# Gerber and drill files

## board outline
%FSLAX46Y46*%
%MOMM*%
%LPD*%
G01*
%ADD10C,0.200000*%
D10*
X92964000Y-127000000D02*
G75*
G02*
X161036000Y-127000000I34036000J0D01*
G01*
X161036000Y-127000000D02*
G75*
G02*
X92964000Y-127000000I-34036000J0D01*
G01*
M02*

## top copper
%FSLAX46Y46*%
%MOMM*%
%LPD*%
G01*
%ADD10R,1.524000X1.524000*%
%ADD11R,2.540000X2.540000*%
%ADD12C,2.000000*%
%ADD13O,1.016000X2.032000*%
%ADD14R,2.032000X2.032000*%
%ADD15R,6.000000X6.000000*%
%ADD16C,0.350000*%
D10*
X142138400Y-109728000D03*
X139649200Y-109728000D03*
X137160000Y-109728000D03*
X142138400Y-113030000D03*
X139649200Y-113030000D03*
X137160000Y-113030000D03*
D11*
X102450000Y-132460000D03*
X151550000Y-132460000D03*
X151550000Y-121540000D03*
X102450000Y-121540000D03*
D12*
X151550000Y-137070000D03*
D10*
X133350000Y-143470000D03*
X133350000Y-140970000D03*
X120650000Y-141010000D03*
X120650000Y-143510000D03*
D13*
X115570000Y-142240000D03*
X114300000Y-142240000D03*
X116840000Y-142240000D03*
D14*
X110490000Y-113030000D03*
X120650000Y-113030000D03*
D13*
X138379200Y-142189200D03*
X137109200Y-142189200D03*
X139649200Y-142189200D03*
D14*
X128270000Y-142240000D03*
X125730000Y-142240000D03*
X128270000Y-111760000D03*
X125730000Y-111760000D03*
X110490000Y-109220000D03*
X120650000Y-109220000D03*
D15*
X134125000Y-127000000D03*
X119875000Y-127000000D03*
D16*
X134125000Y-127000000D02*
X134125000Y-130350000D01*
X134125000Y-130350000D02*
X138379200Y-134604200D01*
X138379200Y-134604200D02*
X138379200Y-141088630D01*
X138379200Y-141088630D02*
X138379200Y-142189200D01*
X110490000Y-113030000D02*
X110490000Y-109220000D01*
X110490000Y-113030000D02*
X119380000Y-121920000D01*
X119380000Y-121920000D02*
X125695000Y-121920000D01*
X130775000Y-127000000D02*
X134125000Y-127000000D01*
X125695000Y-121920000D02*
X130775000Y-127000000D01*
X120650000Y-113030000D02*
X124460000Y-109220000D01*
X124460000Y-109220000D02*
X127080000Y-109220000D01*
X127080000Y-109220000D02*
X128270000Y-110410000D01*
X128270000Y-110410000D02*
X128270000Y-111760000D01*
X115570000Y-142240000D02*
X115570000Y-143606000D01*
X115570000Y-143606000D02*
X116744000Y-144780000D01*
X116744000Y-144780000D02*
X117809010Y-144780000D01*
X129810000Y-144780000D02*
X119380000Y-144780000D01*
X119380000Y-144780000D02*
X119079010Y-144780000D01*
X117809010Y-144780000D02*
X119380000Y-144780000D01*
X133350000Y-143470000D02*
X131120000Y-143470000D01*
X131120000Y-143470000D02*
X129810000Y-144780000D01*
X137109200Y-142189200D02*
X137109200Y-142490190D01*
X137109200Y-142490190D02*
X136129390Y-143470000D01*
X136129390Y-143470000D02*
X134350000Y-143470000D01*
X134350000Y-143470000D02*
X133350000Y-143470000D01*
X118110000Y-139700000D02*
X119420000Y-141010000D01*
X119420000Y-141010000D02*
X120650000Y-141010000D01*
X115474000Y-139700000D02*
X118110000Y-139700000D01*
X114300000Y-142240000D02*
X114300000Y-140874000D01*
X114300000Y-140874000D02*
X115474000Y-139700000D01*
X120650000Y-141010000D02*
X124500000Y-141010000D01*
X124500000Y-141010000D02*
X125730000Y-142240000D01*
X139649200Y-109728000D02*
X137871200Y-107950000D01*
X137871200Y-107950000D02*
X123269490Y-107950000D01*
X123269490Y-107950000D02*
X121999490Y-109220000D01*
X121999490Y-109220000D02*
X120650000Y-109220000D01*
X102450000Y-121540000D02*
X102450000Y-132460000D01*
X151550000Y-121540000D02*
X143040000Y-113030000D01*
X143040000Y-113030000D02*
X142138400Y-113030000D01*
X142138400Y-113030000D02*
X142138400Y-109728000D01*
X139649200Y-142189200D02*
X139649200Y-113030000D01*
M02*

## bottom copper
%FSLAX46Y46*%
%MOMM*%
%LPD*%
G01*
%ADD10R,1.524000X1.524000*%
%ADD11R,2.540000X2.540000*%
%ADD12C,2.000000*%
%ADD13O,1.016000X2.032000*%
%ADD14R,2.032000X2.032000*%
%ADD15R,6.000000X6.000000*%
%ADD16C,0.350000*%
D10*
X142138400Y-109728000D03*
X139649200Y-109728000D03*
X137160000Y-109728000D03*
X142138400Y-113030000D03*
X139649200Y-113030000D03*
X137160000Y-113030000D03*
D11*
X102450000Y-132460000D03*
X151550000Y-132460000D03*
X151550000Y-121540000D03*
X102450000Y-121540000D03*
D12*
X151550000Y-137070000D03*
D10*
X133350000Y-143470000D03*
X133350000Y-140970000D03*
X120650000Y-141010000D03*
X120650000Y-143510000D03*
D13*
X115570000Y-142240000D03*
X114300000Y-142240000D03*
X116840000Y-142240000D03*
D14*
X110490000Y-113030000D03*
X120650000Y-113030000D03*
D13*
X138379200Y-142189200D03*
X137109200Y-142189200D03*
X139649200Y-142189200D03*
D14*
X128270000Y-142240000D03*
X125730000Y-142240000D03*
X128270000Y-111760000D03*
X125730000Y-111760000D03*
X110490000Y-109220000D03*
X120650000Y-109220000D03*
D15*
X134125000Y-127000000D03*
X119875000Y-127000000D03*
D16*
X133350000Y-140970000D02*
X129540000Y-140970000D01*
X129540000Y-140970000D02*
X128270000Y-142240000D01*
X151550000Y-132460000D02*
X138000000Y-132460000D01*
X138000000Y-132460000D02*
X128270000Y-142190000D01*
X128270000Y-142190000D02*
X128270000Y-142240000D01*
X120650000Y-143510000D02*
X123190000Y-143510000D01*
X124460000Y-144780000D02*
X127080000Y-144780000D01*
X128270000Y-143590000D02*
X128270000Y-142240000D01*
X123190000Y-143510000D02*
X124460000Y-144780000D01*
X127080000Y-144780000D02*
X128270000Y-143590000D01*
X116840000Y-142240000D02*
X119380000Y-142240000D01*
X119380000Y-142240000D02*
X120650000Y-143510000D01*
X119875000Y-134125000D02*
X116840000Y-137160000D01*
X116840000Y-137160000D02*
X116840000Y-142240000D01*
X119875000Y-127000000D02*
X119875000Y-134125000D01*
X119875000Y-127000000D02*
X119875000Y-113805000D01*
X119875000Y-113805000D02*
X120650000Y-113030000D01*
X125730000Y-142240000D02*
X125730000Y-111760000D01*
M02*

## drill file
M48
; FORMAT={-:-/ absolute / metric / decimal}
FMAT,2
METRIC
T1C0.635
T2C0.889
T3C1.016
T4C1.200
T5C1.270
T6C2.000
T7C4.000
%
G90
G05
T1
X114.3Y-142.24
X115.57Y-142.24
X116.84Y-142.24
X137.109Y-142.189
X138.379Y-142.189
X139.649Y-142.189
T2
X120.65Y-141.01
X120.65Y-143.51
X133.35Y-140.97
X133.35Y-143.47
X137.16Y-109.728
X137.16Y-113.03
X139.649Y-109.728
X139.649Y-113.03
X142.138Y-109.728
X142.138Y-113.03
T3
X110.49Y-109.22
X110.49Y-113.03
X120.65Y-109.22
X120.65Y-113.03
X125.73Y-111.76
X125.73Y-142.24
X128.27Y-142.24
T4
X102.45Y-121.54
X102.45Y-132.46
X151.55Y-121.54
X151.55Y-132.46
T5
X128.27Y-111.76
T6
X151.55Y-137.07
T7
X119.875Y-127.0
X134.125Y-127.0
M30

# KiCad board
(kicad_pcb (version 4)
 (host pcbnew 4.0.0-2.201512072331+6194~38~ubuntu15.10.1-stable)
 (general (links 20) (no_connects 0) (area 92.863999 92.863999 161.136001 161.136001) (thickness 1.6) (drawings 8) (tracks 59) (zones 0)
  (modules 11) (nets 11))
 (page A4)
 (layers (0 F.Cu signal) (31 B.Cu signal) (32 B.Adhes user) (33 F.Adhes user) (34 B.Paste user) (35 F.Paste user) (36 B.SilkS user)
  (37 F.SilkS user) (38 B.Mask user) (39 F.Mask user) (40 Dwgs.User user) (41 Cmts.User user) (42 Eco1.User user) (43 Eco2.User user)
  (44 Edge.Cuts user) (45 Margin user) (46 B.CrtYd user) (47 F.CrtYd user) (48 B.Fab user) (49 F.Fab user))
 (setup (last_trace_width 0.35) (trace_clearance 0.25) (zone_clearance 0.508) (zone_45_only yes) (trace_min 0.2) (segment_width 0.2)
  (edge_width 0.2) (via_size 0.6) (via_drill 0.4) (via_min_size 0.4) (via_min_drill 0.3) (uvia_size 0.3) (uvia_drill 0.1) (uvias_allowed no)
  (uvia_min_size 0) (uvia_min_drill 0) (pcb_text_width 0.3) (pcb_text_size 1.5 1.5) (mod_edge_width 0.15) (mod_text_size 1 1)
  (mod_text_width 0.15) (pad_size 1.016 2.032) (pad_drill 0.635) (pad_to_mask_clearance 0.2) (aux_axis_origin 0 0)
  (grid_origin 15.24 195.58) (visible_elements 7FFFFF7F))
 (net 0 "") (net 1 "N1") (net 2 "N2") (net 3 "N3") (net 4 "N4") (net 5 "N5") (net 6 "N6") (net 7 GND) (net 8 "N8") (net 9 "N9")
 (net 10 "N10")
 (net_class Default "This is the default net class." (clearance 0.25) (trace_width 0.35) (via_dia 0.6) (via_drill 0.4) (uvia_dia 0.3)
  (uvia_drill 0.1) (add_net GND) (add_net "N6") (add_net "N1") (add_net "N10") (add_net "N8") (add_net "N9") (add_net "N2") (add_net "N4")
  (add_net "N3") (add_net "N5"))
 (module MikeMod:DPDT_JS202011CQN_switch (layer F.Cu) (at 139.6492 111.379 180)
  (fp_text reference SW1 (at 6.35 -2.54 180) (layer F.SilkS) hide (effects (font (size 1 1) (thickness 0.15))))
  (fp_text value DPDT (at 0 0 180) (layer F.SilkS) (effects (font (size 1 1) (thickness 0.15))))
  (pad 1 thru_hole rect (at -2.4892 1.651 180) (size 1.524 1.524) (drill 0.889) (layers *.Cu F.SilkS F.Mask) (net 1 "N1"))
  (pad 2 thru_hole rect (at 0 1.651 180) (size 1.524 1.524) (drill 0.889) (layers *.Cu F.SilkS F.Mask) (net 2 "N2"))
  (pad 3 thru_hole rect (at 2.4892 1.651 180) (size 1.524 1.524) (drill 0.889) (layers *.Cu F.SilkS F.Mask) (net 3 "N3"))
  (pad 4 thru_hole rect (at -2.4892 -1.651 180) (size 1.524 1.524) (drill 0.889) (layers *.Cu F.SilkS F.Mask) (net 1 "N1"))
  (pad 5 thru_hole rect (at 0 -1.651 180) (size 1.524 1.524) (drill 0.889) (layers *.Cu F.SilkS F.Mask) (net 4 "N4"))
  (pad 6 thru_hole rect (at 2.4892 -1.651 180) (size 1.524 1.524) (drill 0.889) (layers *.Cu F.SilkS F.Mask) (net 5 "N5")))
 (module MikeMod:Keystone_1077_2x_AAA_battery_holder (layer F.Cu) (at 127 127 180)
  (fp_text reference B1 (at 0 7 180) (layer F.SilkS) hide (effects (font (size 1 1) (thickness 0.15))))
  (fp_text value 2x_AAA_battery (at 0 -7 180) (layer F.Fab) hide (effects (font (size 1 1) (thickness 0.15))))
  (pad 1 thru_hole rect (at 24.55 -5.46 180) (size 2.54 2.54) (drill 1.2) (layers *.Cu F.SilkS F.Mask) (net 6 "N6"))
  (pad 2 thru_hole rect (at -24.55 -5.46 180) (size 2.54 2.54) (drill 1.2) (layers *.Cu F.SilkS F.Mask) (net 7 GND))
  (pad 3 thru_hole rect (at -24.55 5.46 180) (size 2.54 2.54) (drill 1.2) (layers *.Cu F.SilkS F.Mask) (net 1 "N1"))
  (pad 4 thru_hole rect (at 24.55 5.46 180) (size 2.54 2.54) (drill 1.2) (layers *.Cu F.SilkS F.Mask) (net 6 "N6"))
  (pad "" thru_hole circle (at -24.55 -10.07 180) (size 2 2) (drill 2) (layers *.Cu)))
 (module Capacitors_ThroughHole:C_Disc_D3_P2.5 (layer F.Cu) (at 133.35 143.47 90)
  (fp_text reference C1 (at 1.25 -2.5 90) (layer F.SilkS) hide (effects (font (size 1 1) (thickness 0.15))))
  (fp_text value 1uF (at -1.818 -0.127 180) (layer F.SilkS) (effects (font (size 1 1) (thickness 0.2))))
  (pad 1 thru_hole rect (at 0 0 90) (size 1.524 1.524) (drill 0.889) (layers *.Cu F.SilkS F.Mask) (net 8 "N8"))
  (pad 2 thru_hole rect (at 2.5 0 90) (size 1.524 1.524) (drill 0.889) (layers *.Cu F.SilkS F.Mask) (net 7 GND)))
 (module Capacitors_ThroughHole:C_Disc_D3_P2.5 (layer F.Cu) (at 120.65 141.01 270)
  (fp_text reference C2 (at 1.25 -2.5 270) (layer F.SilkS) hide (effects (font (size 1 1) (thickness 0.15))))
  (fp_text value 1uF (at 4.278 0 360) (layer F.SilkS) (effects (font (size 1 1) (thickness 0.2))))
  (pad 1 thru_hole rect (at 0 0 270) (size 1.524 1.524) (drill 0.889) (layers *.Cu F.SilkS F.Mask) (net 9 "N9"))
  (pad 2 thru_hole rect (at 2.5 0 270) (size 1.524 1.524) (drill 0.889) (layers *.Cu F.SilkS F.Mask) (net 7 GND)))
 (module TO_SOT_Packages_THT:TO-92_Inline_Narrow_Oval (layer F.Cu) (at 116.84 142.24 180)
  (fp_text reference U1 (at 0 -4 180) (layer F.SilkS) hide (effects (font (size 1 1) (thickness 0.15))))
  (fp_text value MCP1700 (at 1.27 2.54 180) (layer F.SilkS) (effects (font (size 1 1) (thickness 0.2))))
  (pad 2 thru_hole oval (at 1.27 0) (size 1.016 2.032) (drill 0.635) (layers *.Cu F.SilkS F.Mask) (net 8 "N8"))
  (pad 3 thru_hole oval (at 2.54 0) (size 1.016 2.032) (drill 0.635) (layers *.Cu F.SilkS F.Mask) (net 9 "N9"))
  (pad 1 thru_hole oval (at 0 0) (size 1.016 2.032) (drill 0.635) (layers *.Cu F.SilkS F.Mask) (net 7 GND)))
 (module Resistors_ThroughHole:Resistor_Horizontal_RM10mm (layer F.Cu) (at 115.57 113.03)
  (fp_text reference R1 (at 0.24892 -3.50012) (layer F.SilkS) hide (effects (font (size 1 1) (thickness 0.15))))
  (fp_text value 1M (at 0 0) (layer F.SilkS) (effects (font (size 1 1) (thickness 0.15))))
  (pad 1 thru_hole rect (at -5.08 0) (size 2.032 2.032) (drill 1.016) (layers *.Cu F.SilkS F.Mask) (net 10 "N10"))
  (pad 2 thru_hole rect (at 5.08 0) (size 2.032 2.032) (drill 1.016) (layers *.Cu F.SilkS F.Mask) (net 7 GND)))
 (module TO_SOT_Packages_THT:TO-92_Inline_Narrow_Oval (layer F.Cu) (at 139.6492 142.1892 180)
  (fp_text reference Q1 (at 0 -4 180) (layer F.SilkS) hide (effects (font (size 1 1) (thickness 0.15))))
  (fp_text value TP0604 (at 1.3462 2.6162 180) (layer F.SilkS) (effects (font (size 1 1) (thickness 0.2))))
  (pad 2 thru_hole oval (at 1.27 0) (size 1.016 2.032) (drill 0.635) (layers *.Cu F.SilkS F.Mask) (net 10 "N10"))
  (pad 3 thru_hole oval (at 2.54 0) (size 1.016 2.032) (drill 0.635) (layers *.Cu F.SilkS F.Mask) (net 8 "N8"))
  (pad 1 thru_hole oval (at 0 0) (size 1.016 2.032) (drill 0.635) (layers *.Cu F.SilkS F.Mask) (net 4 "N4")))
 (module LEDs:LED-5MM (layer F.Cu) (at 128.27 142.24 180)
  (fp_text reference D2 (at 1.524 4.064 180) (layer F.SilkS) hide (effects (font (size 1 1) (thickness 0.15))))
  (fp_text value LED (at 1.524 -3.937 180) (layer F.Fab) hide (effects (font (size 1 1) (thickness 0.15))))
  (pad 1 thru_hole rect (at 0 0 270) (size 2.032 2.032) (drill 1.016) (layers *.Cu F.SilkS F.Mask) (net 7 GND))
  (pad 2 thru_hole rect (at 2.54 0 180) (size 2.032 2.032) (drill 1.016) (layers *.Cu F.SilkS F.Mask) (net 9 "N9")))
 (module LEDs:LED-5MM (layer F.Cu) (at 128.27 111.76 180)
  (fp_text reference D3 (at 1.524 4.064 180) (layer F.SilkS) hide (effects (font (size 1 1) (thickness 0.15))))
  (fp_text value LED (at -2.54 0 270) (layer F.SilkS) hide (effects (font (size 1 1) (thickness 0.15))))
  (pad 1 thru_hole rect (at 0 0 270) (size 2.032 2.032) (drill 1.27) (layers *.Cu F.SilkS F.Mask) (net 7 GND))
  (pad 2 thru_hole rect (at 2.54 0 180) (size 2.032 2.032) (drill 1.016) (layers *.Cu F.SilkS F.Mask) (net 9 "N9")))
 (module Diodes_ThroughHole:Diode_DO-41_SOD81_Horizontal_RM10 (layer F.Cu) (at 120.65 109.21746 180)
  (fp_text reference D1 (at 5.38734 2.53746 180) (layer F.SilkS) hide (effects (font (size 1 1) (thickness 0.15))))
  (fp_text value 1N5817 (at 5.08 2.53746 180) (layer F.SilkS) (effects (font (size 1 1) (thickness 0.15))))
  (pad 2 thru_hole rect (at 10.16 -0.00254) (size 2.032 2.032) (drill 1.016) (layers *.Cu F.SilkS F.Mask) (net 10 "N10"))
  (pad 1 thru_hole rect (at 0 -0.00254) (size 2.032 2.032) (drill 1.016) (layers *.Cu F.SilkS F.Mask) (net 2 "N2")))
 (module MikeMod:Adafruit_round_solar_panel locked (layer B.Cu) (at 127 127)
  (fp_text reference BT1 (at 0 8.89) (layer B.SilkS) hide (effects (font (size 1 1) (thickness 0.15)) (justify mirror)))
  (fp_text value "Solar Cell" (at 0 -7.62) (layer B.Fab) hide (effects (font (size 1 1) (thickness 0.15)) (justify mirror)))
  (pad 1 thru_hole rect (at 7.125 0) (size 6 6) (drill 4) (layers *.Cu B.SilkS B.Mask) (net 10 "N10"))
  (pad 2 thru_hole rect (at -7.125 0) (size 6 6) (drill 4) (layers *.Cu B.SilkS B.Mask) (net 7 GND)))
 (gr_arc (start 127 127) (end 92.964 127) (angle 180) (layer Edge.Cuts) (width 0.2))
 (gr_arc (start 127 127) (end 161.036 127) (angle 180) (layer Edge.Cuts) (width 0.2))
 (segment (start 134.125 127) (end 134.125 130.35) (width 0.35) (layer F.Cu) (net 10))
 (segment (start 134.125 130.35) (end 138.3792 134.6042) (width 0.35) (layer F.Cu) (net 10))
 (segment (start 138.3792 134.6042) (end 138.3792 141.08863) (width 0.35) (layer F.Cu) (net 10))
 (segment (start 138.3792 141.08863) (end 138.3792 142.1892) (width 0.35) (layer F.Cu) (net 10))
 (segment (start 110.49 113.03) (end 110.49 109.22) (width 0.35) (layer F.Cu) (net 10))
 (segment (start 110.49 113.03) (end 119.38 121.92) (width 0.35) (layer F.Cu) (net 10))
 (segment (start 119.38 121.92) (end 125.695 121.92) (width 0.35) (layer F.Cu) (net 10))
 (segment (start 130.775 127) (end 134.125 127) (width 0.35) (layer F.Cu) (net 10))
 (segment (start 125.695 121.92) (end 130.775 127) (width 0.35) (layer F.Cu) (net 10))
 (segment (start 133.35 140.97) (end 129.54 140.97) (width 0.35) (layer B.Cu) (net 7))
 (segment (start 129.54 140.97) (end 128.27 142.24) (width 0.35) (layer B.Cu) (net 7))
 (segment (start 120.65 113.03) (end 124.46 109.22) (width 0.35) (layer F.Cu) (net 7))
 (segment (start 124.46 109.22) (end 127.08 109.22) (width 0.35) (layer F.Cu) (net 7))
 (segment (start 127.08 109.22) (end 128.27 110.41) (width 0.35) (layer F.Cu) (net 7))
 (segment (start 128.27 110.41) (end 128.27 111.76) (width 0.35) (layer F.Cu) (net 7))
 (segment (start 151.55 132.46) (end 138 132.46) (width 0.35) (layer B.Cu) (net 7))
 (segment (start 138 132.46) (end 128.27 142.19) (width 0.35) (layer B.Cu) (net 7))
 (segment (start 128.27 142.19) (end 128.27 142.24) (width 0.35) (layer B.Cu) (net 7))
 (segment (start 120.65 143.51) (end 123.19 143.51) (width 0.35) (layer B.Cu) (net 7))
 (segment (start 124.46 144.78) (end 127.08 144.78) (width 0.35) (layer B.Cu) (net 7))
 (segment (start 128.27 143.59) (end 128.27 142.24) (width 0.35) (layer B.Cu) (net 7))
 (segment (start 123.19 143.51) (end 124.46 144.78) (width 0.35) (layer B.Cu) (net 7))
 (segment (start 127.08 144.78) (end 128.27 143.59) (width 0.35) (layer B.Cu) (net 7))
 (segment (start 116.84 142.24) (end 119.38 142.24) (width 0.35) (layer B.Cu) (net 7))
 (segment (start 119.38 142.24) (end 120.65 143.51) (width 0.35) (layer B.Cu) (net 7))
 (segment (start 119.875 134.125) (end 116.84 137.16) (width 0.35) (layer B.Cu) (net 7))
 (segment (start 116.84 137.16) (end 116.84 142.24) (width 0.35) (layer B.Cu) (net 7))
 (segment (start 119.875 127) (end 119.875 134.125) (width 0.35) (layer B.Cu) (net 7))
 (segment (start 119.875 127) (end 119.875 113.805) (width 0.35) (layer B.Cu) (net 7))
 (segment (start 119.875 113.805) (end 120.65 113.03) (width 0.35) (layer B.Cu) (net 7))
 (segment (start 115.57 142.24) (end 115.57 143.606) (width 0.35) (layer F.Cu) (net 8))
 (segment (start 115.57 143.606) (end 116.744 144.78) (width 0.35) (layer F.Cu) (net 8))
 (segment (start 116.744 144.78) (end 117.80901 144.78) (width 0.35) (layer F.Cu) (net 8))
 (segment (start 129.81 144.78) (end 119.38 144.78) (width 0.35) (layer F.Cu) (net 8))
 (segment (start 119.38 144.78) (end 119.07901 144.78) (width 0.35) (layer F.Cu) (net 8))
 (segment (start 117.80901 144.78) (end 119.38 144.78) (width 0.35) (layer F.Cu) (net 8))
 (segment (start 133.35 143.47) (end 131.12 143.47) (width 0.35) (layer F.Cu) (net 8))
 (segment (start 131.12 143.47) (end 129.81 144.78) (width 0.35) (layer F.Cu) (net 8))
 (segment (start 137.1092 142.1892) (end 137.1092 142.49019) (width 0.35) (layer F.Cu) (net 8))
 (segment (start 137.1092 142.49019) (end 136.12939 143.47) (width 0.35) (layer F.Cu) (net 8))
 (segment (start 136.12939 143.47) (end 134.35 143.47) (width 0.35) (layer F.Cu) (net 8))
 (segment (start 134.35 143.47) (end 133.35 143.47) (width 0.35) (layer F.Cu) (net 8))
 (segment (start 118.11 139.7) (end 119.42 141.01) (width 0.35) (layer F.Cu) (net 9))
 (segment (start 119.42 141.01) (end 120.65 141.01) (width 0.35) (layer F.Cu) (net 9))
 (segment (start 115.474 139.7) (end 118.11 139.7) (width 0.35) (layer F.Cu) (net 9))
 (segment (start 114.3 142.24) (end 114.3 140.874) (width 0.35) (layer F.Cu) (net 9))
 (segment (start 114.3 140.874) (end 115.474 139.7) (width 0.35) (layer F.Cu) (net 9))
 (segment (start 120.65 141.01) (end 124.5 141.01) (width 0.35) (layer F.Cu) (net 9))
 (segment (start 125.73 142.24) (end 125.73 111.76) (width 0.35) (layer B.Cu) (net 9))
 (segment (start 124.5 141.01) (end 125.73 142.24) (width 0.35) (layer F.Cu) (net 9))
 (segment (start 139.6492 109.728) (end 137.8712 107.95) (width 0.35) (layer F.Cu) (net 2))
 (segment (start 137.8712 107.95) (end 123.26949 107.95) (width 0.35) (layer F.Cu) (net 2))
 (segment (start 123.26949 107.95) (end 121.99949 109.22) (width 0.35) (layer F.Cu) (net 2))
 (segment (start 121.99949 109.22) (end 120.65 109.22) (width 0.35) (layer F.Cu) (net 2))
 (segment (start 102.45 121.54) (end 102.45 132.46) (width 0.35) (layer F.Cu) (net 6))
 (segment (start 151.55 121.54) (end 143.04 113.03) (width 0.35) (layer F.Cu) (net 1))
 (segment (start 143.04 113.03) (end 142.1384 113.03) (width 0.35) (layer F.Cu) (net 1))
 (segment (start 142.1384 113.03) (end 142.1384 109.728) (width 0.35) (layer F.Cu) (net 1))
 (segment (start 139.6492 142.1892) (end 139.6492 113.03) (width 0.35) (layer F.Cu) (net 4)))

